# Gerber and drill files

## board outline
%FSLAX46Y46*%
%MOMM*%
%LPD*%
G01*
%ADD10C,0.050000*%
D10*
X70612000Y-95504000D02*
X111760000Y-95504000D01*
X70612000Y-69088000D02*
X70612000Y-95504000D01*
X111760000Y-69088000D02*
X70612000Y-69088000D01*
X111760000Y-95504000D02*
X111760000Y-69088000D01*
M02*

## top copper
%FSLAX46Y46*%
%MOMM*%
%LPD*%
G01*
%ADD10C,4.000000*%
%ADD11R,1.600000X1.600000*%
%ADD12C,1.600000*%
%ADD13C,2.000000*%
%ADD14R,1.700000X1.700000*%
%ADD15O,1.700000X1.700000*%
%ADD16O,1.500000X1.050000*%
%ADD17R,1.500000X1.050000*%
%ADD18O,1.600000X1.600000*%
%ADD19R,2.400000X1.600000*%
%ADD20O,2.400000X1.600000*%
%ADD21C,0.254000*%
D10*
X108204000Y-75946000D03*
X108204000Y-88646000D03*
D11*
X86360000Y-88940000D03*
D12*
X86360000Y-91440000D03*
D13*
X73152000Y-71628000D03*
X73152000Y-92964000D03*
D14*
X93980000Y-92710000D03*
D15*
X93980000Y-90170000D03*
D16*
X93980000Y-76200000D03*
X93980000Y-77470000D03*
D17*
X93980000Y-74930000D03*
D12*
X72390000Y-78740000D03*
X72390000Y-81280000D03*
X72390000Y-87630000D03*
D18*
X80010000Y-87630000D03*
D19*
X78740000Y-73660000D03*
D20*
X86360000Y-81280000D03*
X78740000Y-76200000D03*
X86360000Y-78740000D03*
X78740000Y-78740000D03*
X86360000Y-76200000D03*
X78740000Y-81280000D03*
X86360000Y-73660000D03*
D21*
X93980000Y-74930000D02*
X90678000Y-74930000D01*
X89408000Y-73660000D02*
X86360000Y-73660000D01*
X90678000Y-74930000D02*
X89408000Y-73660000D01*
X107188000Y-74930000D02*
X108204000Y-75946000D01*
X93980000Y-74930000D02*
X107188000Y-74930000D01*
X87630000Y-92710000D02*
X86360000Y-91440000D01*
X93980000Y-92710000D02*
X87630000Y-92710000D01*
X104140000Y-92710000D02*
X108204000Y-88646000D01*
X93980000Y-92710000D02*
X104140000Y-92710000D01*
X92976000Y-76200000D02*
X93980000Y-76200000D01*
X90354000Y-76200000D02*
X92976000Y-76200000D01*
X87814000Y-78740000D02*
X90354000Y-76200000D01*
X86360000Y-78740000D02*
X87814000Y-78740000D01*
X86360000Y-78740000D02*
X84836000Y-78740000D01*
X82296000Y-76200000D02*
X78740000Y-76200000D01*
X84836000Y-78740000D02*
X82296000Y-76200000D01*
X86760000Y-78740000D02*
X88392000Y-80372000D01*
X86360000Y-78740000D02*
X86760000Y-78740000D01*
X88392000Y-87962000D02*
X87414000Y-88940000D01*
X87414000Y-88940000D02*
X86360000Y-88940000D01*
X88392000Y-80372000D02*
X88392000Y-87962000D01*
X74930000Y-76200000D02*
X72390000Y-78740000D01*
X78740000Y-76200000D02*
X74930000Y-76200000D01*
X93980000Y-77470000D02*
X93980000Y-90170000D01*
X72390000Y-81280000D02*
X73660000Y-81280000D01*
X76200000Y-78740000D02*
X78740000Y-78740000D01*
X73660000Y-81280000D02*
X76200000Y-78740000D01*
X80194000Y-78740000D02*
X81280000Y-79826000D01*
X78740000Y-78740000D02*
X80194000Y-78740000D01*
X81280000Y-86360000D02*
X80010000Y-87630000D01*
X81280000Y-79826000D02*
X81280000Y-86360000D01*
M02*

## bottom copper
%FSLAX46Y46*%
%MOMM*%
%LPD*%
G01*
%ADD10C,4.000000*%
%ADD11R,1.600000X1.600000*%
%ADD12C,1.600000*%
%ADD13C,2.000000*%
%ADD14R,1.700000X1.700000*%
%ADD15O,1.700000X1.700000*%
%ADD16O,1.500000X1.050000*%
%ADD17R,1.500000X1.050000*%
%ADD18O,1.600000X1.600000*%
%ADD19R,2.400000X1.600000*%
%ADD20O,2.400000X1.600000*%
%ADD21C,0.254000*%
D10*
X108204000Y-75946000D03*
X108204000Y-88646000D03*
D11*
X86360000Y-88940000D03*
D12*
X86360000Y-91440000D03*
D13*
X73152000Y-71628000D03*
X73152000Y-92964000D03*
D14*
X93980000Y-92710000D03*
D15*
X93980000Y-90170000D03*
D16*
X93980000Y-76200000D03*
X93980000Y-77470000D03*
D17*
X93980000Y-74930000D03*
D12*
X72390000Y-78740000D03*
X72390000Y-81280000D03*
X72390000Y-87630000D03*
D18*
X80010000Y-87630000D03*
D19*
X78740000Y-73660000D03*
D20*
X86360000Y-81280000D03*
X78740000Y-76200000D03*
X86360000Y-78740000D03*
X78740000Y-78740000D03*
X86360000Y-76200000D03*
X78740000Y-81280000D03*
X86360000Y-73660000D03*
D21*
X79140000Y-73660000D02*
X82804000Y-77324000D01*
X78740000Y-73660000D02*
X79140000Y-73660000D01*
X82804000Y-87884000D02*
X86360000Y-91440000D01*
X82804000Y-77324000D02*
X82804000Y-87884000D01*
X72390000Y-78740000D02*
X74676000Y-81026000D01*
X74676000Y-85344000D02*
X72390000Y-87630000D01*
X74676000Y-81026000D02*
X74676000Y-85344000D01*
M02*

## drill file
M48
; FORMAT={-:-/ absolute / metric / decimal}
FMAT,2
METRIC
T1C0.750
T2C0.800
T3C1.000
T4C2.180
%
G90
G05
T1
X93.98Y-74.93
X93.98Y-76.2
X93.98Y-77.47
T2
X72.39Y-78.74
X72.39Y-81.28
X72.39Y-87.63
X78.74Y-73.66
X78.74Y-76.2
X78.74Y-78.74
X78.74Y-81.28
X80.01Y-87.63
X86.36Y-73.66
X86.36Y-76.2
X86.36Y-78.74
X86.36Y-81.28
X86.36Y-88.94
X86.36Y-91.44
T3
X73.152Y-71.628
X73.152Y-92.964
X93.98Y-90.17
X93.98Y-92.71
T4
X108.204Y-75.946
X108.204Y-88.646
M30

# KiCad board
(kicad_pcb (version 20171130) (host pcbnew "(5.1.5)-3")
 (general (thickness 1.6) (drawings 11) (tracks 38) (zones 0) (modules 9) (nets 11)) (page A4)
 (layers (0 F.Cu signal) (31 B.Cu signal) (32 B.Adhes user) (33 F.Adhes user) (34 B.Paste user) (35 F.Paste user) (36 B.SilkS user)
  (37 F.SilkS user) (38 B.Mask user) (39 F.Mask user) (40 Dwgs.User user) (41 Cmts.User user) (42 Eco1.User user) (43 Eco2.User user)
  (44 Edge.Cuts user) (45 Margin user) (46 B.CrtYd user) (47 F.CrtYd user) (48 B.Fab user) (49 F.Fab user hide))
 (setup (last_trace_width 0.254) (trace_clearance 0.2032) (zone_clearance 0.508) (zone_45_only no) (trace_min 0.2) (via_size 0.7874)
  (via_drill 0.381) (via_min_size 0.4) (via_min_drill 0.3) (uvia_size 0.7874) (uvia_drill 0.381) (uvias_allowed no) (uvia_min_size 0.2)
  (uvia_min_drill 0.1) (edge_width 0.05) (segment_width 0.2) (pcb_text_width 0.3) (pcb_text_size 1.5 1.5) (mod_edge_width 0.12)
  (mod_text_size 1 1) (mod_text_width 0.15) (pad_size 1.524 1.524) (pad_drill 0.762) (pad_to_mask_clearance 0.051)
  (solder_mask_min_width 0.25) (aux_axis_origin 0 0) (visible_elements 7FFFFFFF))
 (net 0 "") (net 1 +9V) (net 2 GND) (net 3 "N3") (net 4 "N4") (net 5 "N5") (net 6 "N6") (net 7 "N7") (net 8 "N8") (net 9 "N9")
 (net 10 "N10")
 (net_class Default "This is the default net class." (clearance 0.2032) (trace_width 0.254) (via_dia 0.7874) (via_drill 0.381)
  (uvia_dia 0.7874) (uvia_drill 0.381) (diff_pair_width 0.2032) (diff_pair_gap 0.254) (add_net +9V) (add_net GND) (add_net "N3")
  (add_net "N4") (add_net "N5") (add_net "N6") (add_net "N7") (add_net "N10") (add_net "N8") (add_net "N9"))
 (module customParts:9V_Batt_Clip (layer F.Cu) (at 108.204 82.296 270)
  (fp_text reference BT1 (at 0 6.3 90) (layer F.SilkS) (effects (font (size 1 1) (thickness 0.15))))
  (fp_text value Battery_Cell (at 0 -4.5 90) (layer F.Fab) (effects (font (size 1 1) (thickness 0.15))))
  (pad 1 thru_hole circle (at -6.35 0 270) (size 4 4) (drill 2.18) (layers *.Cu *.Mask) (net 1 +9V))
  (pad 2 thru_hole circle (at 6.35 0 270) (size 4 4) (drill 2.18) (layers *.Cu *.Mask) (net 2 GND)))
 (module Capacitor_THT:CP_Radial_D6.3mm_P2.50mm (layer F.Cu) (at 86.36 88.94 270)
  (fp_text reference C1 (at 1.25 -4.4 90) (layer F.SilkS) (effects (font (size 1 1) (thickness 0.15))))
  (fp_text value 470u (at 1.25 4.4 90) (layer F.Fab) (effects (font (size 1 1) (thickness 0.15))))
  (pad 1 thru_hole rect (at 0 0 270) (size 1.6 1.6) (drill 0.8) (layers *.Cu *.Mask) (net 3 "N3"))
  (pad 2 thru_hole circle (at 2.5 0 270) (size 1.6 1.6) (drill 0.8) (layers *.Cu *.Mask) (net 2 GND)))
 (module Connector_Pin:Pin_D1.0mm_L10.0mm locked (layer B.Cu) (at 73.152 71.628)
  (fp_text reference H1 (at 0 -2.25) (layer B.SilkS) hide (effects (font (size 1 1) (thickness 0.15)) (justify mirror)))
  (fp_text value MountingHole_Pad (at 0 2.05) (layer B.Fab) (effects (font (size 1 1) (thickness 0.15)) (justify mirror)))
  (pad 1 thru_hole circle (at 0 0) (size 2 2) (drill 1) (layers *.Cu *.Mask) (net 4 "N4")))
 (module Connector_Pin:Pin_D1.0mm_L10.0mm (layer B.Cu) (at 73.152 92.964)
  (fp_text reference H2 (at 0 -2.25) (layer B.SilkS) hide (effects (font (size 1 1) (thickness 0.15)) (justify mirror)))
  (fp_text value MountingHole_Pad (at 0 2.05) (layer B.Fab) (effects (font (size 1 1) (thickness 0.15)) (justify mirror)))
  (pad 1 thru_hole circle (at 0 0) (size 2 2) (drill 1) (layers *.Cu *.Mask) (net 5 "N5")))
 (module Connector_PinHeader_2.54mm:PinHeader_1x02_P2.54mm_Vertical (layer B.Cu) (at 93.98 92.71)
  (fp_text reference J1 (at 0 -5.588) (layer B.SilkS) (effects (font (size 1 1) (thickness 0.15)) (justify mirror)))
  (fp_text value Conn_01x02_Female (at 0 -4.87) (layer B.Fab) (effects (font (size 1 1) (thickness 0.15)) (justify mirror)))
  (pad 1 thru_hole rect (at 0 0) (size 1.7 1.7) (drill 1) (layers *.Cu *.Mask) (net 2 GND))
  (pad 2 thru_hole oval (at 0 -2.54) (size 1.7 1.7) (drill 1) (layers *.Cu *.Mask) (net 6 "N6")))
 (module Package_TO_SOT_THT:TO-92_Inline (layer F.Cu) (at 93.98 74.93 270)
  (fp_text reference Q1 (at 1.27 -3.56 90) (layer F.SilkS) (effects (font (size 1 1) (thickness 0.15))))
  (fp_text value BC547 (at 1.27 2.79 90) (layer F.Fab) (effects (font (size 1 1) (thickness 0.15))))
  (pad 2 thru_hole oval (at 1.27 0 270) (size 1.05 1.5) (drill 0.75) (layers *.Cu *.Mask) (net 3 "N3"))
  (pad 3 thru_hole oval (at 2.54 0 270) (size 1.05 1.5) (drill 0.75) (layers *.Cu *.Mask) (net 6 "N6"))
  (pad 1 thru_hole rect (at 0 0 270) (size 1.05 1.5) (drill 0.75) (layers *.Cu *.Mask) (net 1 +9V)))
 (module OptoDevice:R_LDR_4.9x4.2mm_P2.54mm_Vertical (layer F.Cu) (at 72.39 78.74 270)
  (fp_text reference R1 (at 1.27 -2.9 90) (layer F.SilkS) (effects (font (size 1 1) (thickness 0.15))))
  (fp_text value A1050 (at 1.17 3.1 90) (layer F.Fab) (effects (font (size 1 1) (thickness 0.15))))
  (pad 1 thru_hole circle (at 0 0 270) (size 1.6 1.6) (drill 0.8) (layers *.Cu *.Mask) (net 3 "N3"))
  (pad 2 thru_hole circle (at 2.54 0 270) (size 1.6 1.6) (drill 0.8) (layers *.Cu *.Mask) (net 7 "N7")))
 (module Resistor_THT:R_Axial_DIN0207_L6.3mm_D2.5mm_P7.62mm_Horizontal (layer F.Cu) (at 72.39 87.63)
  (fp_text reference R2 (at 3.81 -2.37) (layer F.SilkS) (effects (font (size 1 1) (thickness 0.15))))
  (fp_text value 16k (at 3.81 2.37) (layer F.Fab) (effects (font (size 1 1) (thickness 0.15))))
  (pad 1 thru_hole circle (at 0 0) (size 1.6 1.6) (drill 0.8) (layers *.Cu *.Mask) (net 3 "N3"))
  (pad 2 thru_hole oval (at 7.62 0) (size 1.6 1.6) (drill 0.8) (layers *.Cu *.Mask) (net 7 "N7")))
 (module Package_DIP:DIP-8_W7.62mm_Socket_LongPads (layer F.Cu) (at 78.74 73.66)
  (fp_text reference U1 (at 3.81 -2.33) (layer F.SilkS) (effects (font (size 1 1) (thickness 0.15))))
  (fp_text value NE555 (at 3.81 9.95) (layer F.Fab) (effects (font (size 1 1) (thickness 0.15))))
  (pad 1 thru_hole rect (at 0 0) (size 2.4 1.6) (drill 0.8) (layers *.Cu *.Mask) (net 2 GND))
  (pad 5 thru_hole oval (at 7.62 7.62) (size 2.4 1.6) (drill 0.8) (layers *.Cu *.Mask) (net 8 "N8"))
  (pad 2 thru_hole oval (at 0 2.54) (size 2.4 1.6) (drill 0.8) (layers *.Cu *.Mask) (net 3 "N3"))
  (pad 6 thru_hole oval (at 7.62 5.08) (size 2.4 1.6) (drill 0.8) (layers *.Cu *.Mask) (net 3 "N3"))
  (pad 3 thru_hole oval (at 0 5.08) (size 2.4 1.6) (drill 0.8) (layers *.Cu *.Mask) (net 7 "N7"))
  (pad 7 thru_hole oval (at 7.62 2.54) (size 2.4 1.6) (drill 0.8) (layers *.Cu *.Mask) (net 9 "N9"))
  (pad 4 thru_hole oval (at 0 7.62) (size 2.4 1.6) (drill 0.8) (layers *.Cu *.Mask) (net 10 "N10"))
  (pad 8 thru_hole oval (at 7.62 0) (size 2.4 1.6) (drill 0.8) (layers *.Cu *.Mask) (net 1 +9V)))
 (gr_line (start 70.612 95.504) (end 111.76 95.504) (layer Edge.Cuts) (width 0.05))
 (gr_line (start 70.612 69.088) (end 70.612 95.504) (layer Edge.Cuts) (width 0.05))
 (gr_line (start 111.76 69.088) (end 70.612 69.088) (layer Edge.Cuts) (width 0.05))
 (gr_line (start 111.76 95.504) (end 111.76 69.088) (layer Edge.Cuts) (width 0.05))
 (segment (start 93.98 74.93) (end 90.678 74.93) (width 0.254) (layer F.Cu) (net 1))
 (segment (start 89.408 73.66) (end 86.36 73.66) (width 0.254) (layer F.Cu) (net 1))
 (segment (start 90.678 74.93) (end 89.408 73.66) (width 0.254) (layer F.Cu) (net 1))
 (segment (start 107.188 74.93) (end 108.204 75.946) (width 0.254) (layer F.Cu) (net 1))
 (segment (start 93.98 74.93) (end 107.188 74.93) (width 0.254) (layer F.Cu) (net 1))
 (segment (start 79.14 73.66) (end 82.804 77.324) (width 0.254) (layer B.Cu) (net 2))
 (segment (start 78.74 73.66) (end 79.14 73.66) (width 0.254) (layer B.Cu) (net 2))
 (segment (start 82.804 87.884) (end 86.36 91.44) (width 0.254) (layer B.Cu) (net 2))
 (segment (start 82.804 77.324) (end 82.804 87.884) (width 0.254) (layer B.Cu) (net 2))
 (segment (start 87.63 92.71) (end 86.36 91.44) (width 0.254) (layer F.Cu) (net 2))
 (segment (start 93.98 92.71) (end 87.63 92.71) (width 0.254) (layer F.Cu) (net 2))
 (segment (start 104.14 92.71) (end 108.204 88.646) (width 0.254) (layer F.Cu) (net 2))
 (segment (start 93.98 92.71) (end 104.14 92.71) (width 0.254) (layer F.Cu) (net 2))
 (segment (start 92.976 76.2) (end 93.98 76.2) (width 0.254) (layer F.Cu) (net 3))
 (segment (start 90.354 76.2) (end 92.976 76.2) (width 0.254) (layer F.Cu) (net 3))
 (segment (start 87.814 78.74) (end 90.354 76.2) (width 0.254) (layer F.Cu) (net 3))
 (segment (start 86.36 78.74) (end 87.814 78.74) (width 0.254) (layer F.Cu) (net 3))
 (segment (start 86.36 78.74) (end 84.836 78.74) (width 0.254) (layer F.Cu) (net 3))
 (segment (start 82.296 76.2) (end 78.74 76.2) (width 0.254) (layer F.Cu) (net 3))
 (segment (start 84.836 78.74) (end 82.296 76.2) (width 0.254) (layer F.Cu) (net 3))
 (segment (start 86.76 78.74) (end 88.392 80.372) (width 0.254) (layer F.Cu) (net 3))
 (segment (start 86.36 78.74) (end 86.76 78.74) (width 0.254) (layer F.Cu) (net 3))
 (segment (start 88.392 87.962) (end 87.414 88.94) (width 0.254) (layer F.Cu) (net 3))
 (segment (start 87.414 88.94) (end 86.36 88.94) (width 0.254) (layer F.Cu) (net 3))
 (segment (start 88.392 80.372) (end 88.392 87.962) (width 0.254) (layer F.Cu) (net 3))
 (segment (start 74.93 76.2) (end 72.39 78.74) (width 0.254) (layer F.Cu) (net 3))
 (segment (start 78.74 76.2) (end 74.93 76.2) (width 0.254) (layer F.Cu) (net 3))
 (segment (start 72.39 78.74) (end 74.676 81.026) (width 0.254) (layer B.Cu) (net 3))
 (segment (start 74.676 85.344) (end 72.39 87.63) (width 0.254) (layer B.Cu) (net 3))
 (segment (start 74.676 81.026) (end 74.676 85.344) (width 0.254) (layer B.Cu) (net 3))
 (segment (start 93.98 77.47) (end 93.98 90.17) (width 0.254) (layer F.Cu) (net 6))
 (segment (start 72.39 81.28) (end 73.66 81.28) (width 0.254) (layer F.Cu) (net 7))
 (segment (start 76.2 78.74) (end 78.74 78.74) (width 0.254) (layer F.Cu) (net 7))
 (segment (start 73.66 81.28) (end 76.2 78.74) (width 0.254) (layer F.Cu) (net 7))
 (segment (start 80.194 78.74) (end 81.28 79.826) (width 0.254) (layer F.Cu) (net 7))
 (segment (start 78.74 78.74) (end 80.194 78.74) (width 0.254) (layer F.Cu) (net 7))
 (segment (start 81.28 86.36) (end 80.01 87.63) (width 0.254) (layer F.Cu) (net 7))
 (segment (start 81.28 79.826) (end 81.28 86.36) (width 0.254) (layer F.Cu) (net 7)))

